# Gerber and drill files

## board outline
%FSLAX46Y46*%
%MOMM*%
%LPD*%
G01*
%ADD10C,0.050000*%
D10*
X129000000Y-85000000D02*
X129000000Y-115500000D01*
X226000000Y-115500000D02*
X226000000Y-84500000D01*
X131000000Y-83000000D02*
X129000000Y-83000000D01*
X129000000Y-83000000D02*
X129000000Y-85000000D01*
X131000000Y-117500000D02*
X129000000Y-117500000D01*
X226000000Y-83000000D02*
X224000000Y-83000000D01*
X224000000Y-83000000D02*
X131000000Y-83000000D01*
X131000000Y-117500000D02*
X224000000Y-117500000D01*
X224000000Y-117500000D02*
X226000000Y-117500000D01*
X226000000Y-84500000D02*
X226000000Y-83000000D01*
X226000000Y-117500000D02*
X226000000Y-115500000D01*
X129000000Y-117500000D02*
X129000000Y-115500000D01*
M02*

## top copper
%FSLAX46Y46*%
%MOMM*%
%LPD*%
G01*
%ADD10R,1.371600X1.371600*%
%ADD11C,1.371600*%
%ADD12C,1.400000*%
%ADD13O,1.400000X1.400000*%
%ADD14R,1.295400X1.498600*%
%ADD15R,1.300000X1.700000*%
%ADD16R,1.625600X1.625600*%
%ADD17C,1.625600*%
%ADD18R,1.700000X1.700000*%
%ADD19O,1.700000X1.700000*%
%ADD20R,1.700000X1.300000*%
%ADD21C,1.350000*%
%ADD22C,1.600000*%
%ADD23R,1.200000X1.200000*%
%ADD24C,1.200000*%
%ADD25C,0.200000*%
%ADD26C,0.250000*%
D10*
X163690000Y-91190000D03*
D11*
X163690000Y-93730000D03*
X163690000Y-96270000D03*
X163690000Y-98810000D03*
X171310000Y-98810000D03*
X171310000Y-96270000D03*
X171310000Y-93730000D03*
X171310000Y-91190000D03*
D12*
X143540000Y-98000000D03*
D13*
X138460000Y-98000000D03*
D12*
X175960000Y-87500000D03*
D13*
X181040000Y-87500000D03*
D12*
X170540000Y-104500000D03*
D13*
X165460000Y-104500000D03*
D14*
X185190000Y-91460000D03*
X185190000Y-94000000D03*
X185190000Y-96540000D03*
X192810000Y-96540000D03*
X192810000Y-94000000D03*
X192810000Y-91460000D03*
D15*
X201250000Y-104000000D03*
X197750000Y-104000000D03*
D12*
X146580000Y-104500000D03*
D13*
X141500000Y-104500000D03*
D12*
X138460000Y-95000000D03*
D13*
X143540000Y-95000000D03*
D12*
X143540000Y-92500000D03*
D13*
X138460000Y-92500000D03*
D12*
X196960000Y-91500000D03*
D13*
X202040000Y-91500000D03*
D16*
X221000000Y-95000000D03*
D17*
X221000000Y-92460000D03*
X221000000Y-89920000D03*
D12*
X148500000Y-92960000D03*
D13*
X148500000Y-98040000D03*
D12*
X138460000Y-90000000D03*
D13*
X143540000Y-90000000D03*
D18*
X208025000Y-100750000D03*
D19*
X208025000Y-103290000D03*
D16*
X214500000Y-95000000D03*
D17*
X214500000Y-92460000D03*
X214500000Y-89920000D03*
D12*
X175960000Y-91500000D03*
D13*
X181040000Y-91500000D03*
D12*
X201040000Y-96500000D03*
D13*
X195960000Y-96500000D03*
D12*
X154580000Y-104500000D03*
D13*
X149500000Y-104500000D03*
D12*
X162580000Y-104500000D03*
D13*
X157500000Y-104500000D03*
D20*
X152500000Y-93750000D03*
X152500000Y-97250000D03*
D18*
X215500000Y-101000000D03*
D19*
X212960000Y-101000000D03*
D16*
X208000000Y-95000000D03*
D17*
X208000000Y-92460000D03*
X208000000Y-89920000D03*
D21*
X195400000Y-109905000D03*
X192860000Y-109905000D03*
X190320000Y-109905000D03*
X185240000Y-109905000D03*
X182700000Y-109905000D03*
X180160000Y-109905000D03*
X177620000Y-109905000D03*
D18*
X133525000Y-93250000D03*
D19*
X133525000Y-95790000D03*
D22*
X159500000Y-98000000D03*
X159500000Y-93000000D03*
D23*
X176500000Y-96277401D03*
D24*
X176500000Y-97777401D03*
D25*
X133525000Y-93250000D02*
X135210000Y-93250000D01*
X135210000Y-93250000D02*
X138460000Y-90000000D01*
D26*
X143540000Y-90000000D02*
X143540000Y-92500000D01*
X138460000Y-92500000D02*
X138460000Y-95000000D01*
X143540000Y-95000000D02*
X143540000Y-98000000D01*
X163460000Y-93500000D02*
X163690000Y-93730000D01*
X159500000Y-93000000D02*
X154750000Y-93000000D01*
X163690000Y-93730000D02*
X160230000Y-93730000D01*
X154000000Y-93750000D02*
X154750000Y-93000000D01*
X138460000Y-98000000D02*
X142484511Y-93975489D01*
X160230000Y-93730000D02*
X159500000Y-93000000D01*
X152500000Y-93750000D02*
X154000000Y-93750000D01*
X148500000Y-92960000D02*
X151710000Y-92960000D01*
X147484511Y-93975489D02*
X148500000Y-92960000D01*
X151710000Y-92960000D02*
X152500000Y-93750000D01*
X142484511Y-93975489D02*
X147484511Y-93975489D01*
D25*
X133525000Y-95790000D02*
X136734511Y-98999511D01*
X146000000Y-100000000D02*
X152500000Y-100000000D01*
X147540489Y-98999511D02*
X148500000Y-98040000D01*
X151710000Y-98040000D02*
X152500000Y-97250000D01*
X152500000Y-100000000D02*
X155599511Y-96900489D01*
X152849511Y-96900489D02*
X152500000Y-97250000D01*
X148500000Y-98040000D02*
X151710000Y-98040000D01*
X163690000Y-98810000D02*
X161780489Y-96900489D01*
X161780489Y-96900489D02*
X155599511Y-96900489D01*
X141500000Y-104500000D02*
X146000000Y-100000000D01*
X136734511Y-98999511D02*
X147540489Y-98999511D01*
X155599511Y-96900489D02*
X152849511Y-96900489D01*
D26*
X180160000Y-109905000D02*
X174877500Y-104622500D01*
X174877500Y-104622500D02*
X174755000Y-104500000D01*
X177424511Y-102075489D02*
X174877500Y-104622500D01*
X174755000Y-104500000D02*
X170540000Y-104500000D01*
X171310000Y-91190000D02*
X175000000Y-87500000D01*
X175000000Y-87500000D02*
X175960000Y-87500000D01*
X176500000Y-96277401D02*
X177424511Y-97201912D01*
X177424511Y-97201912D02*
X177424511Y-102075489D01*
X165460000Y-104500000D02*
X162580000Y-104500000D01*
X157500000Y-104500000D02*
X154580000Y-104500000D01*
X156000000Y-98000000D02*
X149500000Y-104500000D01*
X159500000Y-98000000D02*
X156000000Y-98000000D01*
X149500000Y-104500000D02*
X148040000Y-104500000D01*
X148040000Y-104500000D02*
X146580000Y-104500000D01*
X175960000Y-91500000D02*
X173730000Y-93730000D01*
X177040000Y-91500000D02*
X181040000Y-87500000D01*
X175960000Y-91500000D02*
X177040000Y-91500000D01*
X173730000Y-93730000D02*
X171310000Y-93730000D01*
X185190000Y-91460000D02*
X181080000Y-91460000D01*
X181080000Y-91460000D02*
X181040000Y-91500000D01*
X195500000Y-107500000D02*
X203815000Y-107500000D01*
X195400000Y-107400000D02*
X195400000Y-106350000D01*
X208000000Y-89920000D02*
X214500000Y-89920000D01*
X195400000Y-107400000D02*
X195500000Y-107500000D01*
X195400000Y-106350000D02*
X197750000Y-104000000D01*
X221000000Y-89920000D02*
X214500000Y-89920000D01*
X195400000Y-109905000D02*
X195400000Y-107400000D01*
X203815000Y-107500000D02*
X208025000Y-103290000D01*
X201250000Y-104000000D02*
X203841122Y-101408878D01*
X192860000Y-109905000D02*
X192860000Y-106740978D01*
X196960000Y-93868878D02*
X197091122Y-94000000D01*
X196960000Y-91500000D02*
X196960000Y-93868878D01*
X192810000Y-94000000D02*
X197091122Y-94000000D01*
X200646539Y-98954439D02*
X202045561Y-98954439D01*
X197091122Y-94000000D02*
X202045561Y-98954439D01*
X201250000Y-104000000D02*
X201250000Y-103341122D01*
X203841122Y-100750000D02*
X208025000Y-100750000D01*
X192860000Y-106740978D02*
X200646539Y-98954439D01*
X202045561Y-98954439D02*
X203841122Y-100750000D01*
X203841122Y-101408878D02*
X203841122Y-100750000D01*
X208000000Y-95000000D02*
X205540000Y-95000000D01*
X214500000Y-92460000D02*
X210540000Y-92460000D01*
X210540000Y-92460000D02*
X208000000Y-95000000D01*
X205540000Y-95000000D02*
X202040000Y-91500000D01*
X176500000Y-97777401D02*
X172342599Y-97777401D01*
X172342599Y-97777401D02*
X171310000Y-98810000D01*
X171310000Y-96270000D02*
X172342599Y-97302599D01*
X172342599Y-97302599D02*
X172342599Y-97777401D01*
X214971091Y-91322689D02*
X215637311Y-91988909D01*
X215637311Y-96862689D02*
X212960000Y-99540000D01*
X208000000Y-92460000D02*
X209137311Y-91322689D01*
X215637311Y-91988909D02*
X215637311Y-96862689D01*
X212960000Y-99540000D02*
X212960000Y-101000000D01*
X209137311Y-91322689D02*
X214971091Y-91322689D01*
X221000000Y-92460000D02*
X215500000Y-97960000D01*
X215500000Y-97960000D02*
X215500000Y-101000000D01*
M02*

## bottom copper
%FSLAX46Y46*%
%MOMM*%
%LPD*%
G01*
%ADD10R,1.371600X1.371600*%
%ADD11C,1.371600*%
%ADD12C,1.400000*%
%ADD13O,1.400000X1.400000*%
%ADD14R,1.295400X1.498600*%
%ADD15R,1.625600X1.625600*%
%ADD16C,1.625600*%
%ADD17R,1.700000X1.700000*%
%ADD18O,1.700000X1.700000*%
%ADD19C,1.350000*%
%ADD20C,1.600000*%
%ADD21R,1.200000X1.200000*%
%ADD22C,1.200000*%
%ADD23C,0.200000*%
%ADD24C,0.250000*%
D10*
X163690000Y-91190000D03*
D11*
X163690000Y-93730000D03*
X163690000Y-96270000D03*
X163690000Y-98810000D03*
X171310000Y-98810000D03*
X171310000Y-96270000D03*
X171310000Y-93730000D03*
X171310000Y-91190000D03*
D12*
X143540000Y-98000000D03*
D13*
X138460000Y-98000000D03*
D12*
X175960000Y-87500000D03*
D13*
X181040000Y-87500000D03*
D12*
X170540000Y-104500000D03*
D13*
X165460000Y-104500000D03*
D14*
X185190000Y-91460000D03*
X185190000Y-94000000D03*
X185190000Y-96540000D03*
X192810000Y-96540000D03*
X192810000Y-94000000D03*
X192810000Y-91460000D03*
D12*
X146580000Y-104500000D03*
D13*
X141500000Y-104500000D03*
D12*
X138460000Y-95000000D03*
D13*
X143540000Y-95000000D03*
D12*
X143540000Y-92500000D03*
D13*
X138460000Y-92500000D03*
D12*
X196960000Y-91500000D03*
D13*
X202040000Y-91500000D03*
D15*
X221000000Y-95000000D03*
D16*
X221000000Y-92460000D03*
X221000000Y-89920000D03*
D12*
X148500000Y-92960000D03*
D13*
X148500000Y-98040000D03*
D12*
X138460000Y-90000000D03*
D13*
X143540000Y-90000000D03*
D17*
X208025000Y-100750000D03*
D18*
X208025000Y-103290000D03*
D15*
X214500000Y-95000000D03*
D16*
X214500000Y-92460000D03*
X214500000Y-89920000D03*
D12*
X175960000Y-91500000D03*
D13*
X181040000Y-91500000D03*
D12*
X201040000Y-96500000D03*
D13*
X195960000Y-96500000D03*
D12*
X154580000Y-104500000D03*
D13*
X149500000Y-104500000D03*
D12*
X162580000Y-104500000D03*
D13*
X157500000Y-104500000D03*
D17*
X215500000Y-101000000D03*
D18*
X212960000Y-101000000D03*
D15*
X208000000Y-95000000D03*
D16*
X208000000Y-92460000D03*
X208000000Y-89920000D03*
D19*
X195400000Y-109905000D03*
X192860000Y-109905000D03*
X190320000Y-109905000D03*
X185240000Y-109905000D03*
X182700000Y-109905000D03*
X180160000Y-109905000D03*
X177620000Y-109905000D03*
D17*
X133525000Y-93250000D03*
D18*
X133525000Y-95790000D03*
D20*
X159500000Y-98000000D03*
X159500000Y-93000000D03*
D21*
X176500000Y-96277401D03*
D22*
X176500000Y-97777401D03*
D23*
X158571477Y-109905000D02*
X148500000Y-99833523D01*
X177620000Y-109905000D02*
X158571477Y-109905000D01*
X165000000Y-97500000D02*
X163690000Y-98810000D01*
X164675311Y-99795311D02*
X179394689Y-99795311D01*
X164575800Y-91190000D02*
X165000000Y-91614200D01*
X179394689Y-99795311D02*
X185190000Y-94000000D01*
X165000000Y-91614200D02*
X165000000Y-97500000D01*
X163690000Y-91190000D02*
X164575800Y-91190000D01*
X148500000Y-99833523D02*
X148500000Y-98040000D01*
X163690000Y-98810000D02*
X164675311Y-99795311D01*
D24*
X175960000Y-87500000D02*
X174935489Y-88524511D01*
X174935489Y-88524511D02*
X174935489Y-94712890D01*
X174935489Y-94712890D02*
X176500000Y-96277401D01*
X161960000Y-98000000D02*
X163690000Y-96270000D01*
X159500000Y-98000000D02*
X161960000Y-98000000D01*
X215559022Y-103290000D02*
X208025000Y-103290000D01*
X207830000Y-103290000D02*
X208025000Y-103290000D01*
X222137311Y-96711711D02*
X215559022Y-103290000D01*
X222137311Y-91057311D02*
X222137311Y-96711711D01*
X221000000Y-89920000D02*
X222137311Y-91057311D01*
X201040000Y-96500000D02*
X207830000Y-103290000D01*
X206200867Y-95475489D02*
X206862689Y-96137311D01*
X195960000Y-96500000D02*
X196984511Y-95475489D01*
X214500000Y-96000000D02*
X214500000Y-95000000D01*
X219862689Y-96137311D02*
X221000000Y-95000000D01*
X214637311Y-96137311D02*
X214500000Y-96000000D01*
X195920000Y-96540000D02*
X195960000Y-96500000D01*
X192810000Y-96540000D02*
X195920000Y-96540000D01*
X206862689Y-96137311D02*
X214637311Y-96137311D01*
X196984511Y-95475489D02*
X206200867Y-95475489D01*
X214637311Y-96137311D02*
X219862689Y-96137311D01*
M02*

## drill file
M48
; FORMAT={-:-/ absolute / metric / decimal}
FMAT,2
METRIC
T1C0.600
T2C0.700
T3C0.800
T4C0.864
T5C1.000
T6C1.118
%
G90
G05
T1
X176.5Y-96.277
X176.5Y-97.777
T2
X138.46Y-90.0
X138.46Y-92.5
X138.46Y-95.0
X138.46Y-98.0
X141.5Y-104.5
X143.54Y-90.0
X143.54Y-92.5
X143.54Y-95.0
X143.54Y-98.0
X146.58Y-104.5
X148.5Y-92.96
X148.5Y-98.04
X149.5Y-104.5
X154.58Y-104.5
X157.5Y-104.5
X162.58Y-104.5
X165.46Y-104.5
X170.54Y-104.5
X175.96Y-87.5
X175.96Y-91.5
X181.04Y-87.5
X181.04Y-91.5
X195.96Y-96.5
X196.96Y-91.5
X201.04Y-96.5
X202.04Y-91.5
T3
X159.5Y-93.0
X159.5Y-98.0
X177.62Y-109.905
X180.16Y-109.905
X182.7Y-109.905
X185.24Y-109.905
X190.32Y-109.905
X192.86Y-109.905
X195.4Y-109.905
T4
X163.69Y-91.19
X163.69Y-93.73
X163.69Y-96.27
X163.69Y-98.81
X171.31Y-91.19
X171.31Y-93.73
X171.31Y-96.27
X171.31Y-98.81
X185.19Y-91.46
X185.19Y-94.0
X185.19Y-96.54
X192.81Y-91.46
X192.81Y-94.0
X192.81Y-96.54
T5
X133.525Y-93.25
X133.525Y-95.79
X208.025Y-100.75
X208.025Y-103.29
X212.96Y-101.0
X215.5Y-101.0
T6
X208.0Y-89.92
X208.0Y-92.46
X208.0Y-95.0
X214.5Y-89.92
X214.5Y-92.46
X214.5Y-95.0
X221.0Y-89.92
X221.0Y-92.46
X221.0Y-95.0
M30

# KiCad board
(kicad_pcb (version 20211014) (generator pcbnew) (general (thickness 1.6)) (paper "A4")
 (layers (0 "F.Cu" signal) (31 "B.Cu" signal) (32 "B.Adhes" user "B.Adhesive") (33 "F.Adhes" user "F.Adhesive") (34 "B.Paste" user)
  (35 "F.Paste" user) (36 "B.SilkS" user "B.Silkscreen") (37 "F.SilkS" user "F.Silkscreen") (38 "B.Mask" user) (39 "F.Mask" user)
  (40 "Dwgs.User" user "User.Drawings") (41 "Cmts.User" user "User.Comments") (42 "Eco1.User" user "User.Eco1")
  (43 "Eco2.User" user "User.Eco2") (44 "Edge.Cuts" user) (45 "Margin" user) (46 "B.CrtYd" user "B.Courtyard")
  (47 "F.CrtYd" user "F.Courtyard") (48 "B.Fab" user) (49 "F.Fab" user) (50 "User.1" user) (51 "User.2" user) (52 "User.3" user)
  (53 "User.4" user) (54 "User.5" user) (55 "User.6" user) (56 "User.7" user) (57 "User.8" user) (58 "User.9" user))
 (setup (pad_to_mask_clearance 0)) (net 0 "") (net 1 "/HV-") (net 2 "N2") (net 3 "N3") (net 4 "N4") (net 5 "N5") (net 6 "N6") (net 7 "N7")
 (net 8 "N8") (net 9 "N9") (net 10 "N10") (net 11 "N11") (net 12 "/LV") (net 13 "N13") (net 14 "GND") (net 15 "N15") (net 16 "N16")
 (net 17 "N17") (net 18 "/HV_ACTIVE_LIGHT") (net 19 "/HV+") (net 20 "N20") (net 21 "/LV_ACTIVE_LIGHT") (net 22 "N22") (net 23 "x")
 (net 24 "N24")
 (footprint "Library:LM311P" (layer "F.Cu") (at 163.69 91.19)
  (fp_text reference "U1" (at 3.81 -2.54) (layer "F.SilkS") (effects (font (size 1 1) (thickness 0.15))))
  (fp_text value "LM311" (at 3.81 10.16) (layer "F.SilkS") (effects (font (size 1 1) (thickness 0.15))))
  (pad "1" thru_hole rect (at 0 0) (size 1.3716 1.3716) (drill 0.8636) (layers *.Cu *.Mask) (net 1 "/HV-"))
  (pad "2" thru_hole circle (at 0 2.54) (size 1.3716 1.3716) (drill 0.8636) (layers *.Cu *.Mask) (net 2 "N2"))
  (pad "3" thru_hole circle (at 0 5.08) (size 1.3716 1.3716) (drill 0.8636) (layers *.Cu *.Mask) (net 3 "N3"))
  (pad "4" thru_hole circle (at 0 7.62) (size 1.3716 1.3716) (drill 0.8636) (layers *.Cu *.Mask) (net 1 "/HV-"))
  (pad "5" thru_hole circle (at 7.62 7.62) (size 1.3716 1.3716) (drill 0.8636) (layers *.Cu *.Mask) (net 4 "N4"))
  (pad "6" thru_hole circle (at 7.62 5.08) (size 1.3716 1.3716) (drill 0.8636) (layers *.Cu *.Mask) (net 4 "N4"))
  (pad "7" thru_hole circle (at 7.62 2.54) (size 1.3716 1.3716) (drill 0.8636) (layers *.Cu *.Mask) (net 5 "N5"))
  (pad "8" thru_hole circle (at 7.62 0) (size 1.3716 1.3716) (drill 0.8636) (layers *.Cu *.Mask) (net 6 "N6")))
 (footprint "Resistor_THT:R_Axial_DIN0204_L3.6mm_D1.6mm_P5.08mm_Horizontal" (layer "F.Cu") (at 143.54 98 180)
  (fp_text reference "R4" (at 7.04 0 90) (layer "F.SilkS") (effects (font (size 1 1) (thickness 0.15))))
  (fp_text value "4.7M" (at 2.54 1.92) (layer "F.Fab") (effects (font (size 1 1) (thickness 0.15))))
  (pad "1" thru_hole circle (at 0 0 180) (size 1.4 1.4) (drill 0.7) (layers *.Cu *.Mask) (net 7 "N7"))
  (pad "2" thru_hole oval (at 5.08 0 180) (size 1.4 1.4) (drill 0.7) (layers *.Cu *.Mask) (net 2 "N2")))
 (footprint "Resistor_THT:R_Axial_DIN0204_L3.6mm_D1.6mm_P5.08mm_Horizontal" (layer "F.Cu") (at 175.96 87.5)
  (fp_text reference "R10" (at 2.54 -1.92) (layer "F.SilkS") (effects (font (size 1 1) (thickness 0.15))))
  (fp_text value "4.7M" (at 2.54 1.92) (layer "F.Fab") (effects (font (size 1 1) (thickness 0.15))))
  (pad "1" thru_hole circle (at 0 0) (size 1.4 1.4) (drill 0.7) (layers *.Cu *.Mask) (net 6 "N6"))
  (pad "2" thru_hole oval (at 5.08 0) (size 1.4 1.4) (drill 0.7) (layers *.Cu *.Mask) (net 5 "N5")))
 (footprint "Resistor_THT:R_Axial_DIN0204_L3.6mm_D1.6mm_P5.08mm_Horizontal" (layer "F.Cu") (at 170.54 104.5 180)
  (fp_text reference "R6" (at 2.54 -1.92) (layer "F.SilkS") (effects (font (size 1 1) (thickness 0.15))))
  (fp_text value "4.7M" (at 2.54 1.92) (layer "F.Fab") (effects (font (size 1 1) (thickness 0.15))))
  (pad "1" thru_hole circle (at 0 0 180) (size 1.4 1.4) (drill 0.7) (layers *.Cu *.Mask) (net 6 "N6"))
  (pad "2" thru_hole oval (at 5.08 0 180) (size 1.4 1.4) (drill 0.7) (layers *.Cu *.Mask) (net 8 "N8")))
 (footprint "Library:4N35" (layer "F.Cu") (at 185.19 91.46)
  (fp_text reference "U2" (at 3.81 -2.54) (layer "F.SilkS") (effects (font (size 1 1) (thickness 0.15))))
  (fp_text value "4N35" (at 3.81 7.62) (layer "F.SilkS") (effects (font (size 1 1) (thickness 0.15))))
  (pad "1" thru_hole rect (at 0 0) (size 1.2954 1.4986) (drill 0.8636) (layers *.Cu *.Mask) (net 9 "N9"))
  (pad "2" thru_hole rect (at 0 2.54) (size 1.2954 1.4986) (drill 0.8636) (layers *.Cu *.Mask) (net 1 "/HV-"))
  (pad "3" thru_hole rect (at 0 5.08) (size 1.2954 1.4986) (drill 0.8636) (layers *.Cu *.Mask) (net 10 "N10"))
  (pad "4" thru_hole rect (at 7.62 5.08) (size 1.2954 1.4986) (drill 0.8636) (layers *.Cu *.Mask) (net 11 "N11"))
  (pad "5" thru_hole rect (at 7.62 2.54) (size 1.2954 1.4986) (drill 0.8636) (layers *.Cu *.Mask) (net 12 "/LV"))
  (pad "6" thru_hole rect (at 7.62 0) (size 1.2954 1.4986) (drill 0.8636) (layers *.Cu *.Mask) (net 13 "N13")))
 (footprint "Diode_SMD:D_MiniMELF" (layer "F.Cu") (at 199.5 104 180)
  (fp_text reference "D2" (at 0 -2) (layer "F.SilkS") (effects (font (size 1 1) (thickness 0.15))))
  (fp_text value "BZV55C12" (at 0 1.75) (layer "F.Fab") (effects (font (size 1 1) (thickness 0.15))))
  (pad "1" smd rect (at -1.75 0 180) (size 1.3 1.7) (layers "F.Cu" "F.Paste" "F.Mask") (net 12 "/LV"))
  (pad "2" smd rect (at 1.75 0 180) (size 1.3 1.7) (layers "F.Cu" "F.Paste" "F.Mask") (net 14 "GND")))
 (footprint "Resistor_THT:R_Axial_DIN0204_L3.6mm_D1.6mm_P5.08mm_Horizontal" (layer "F.Cu") (at 146.58 104.5 180)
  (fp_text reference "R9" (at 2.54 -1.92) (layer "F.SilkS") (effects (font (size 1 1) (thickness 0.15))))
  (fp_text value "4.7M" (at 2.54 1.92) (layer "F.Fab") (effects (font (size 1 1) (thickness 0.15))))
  (pad "1" thru_hole circle (at 0 0 180) (size 1.4 1.4) (drill 0.7) (layers *.Cu *.Mask) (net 3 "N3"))
  (pad "2" thru_hole oval (at 5.08 0 180) (size 1.4 1.4) (drill 0.7) (layers *.Cu *.Mask) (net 1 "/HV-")))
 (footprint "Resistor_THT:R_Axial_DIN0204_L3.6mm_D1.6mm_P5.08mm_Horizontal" (layer "F.Cu") (at 138.46 95)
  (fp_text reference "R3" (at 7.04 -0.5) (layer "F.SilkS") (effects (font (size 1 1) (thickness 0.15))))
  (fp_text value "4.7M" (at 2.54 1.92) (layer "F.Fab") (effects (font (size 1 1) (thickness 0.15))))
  (pad "1" thru_hole circle (at 0 0) (size 1.4 1.4) (drill 0.7) (layers *.Cu *.Mask) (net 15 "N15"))
  (pad "2" thru_hole oval (at 5.08 0) (size 1.4 1.4) (drill 0.7) (layers *.Cu *.Mask) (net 7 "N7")))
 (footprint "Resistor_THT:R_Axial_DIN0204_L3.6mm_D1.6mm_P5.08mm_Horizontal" (layer "F.Cu") (at 143.54 92.5 180)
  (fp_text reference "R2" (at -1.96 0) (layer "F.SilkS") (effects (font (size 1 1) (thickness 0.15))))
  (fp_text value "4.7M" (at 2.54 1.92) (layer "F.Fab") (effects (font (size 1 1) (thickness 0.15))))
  (pad "1" thru_hole circle (at 0 0 180) (size 1.4 1.4) (drill 0.7) (layers *.Cu *.Mask) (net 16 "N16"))
  (pad "2" thru_hole oval (at 5.08 0 180) (size 1.4 1.4) (drill 0.7) (layers *.Cu *.Mask) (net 15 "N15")))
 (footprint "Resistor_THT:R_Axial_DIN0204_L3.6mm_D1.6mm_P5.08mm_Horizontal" (layer "F.Cu") (at 196.96 91.5)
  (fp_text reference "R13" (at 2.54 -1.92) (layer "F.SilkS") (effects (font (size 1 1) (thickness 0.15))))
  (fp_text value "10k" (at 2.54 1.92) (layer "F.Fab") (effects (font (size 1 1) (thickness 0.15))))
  (pad "1" thru_hole circle (at 0 0) (size 1.4 1.4) (drill 0.7) (layers *.Cu *.Mask) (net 12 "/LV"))
  (pad "2" thru_hole oval (at 5.08 0) (size 1.4 1.4) (drill 0.7) (layers *.Cu *.Mask) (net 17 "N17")))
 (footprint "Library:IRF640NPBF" (layer "F.Cu") (at 221 95 90)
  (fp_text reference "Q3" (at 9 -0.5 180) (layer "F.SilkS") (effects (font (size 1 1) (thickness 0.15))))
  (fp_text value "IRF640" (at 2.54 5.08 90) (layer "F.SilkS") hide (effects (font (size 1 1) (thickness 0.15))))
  (pad "1" thru_hole rect (at 0 0 90) (size 1.6256 1.6256) (drill 1.1176) (layers *.Cu *.Mask) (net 11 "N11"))
  (pad "2" thru_hole circle (at 2.54 0 90) (size 1.6256 1.6256) (drill 1.1176) (layers *.Cu *.Mask) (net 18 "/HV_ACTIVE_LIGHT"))
  (pad "3" thru_hole circle (at 5.08 0 90) (size 1.6256 1.6256) (drill 1.1176) (layers *.Cu *.Mask) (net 14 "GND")))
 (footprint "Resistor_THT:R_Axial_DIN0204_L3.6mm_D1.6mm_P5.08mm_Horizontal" (layer "F.Cu") (at 148.5 92.96 -90)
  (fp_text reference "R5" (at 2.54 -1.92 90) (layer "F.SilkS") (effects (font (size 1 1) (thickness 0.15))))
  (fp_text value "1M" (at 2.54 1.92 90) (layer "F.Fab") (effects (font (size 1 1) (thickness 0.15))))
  (pad "1" thru_hole circle (at 0 0 270) (size 1.4 1.4) (drill 0.7) (layers *.Cu *.Mask) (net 2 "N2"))
  (pad "2" thru_hole oval (at 5.08 0 270) (size 1.4 1.4) (drill 0.7) (layers *.Cu *.Mask) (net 1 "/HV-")))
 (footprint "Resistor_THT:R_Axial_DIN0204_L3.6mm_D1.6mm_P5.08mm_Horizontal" (layer "F.Cu") (at 138.46 90)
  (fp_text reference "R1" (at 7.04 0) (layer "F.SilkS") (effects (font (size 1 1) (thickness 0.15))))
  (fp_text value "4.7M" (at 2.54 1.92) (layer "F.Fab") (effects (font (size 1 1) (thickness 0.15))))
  (pad "1" thru_hole circle (at 0 0) (size 1.4 1.4) (drill 0.7) (layers *.Cu *.Mask) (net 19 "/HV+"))
  (pad "2" thru_hole oval (at 5.08 0) (size 1.4 1.4) (drill 0.7) (layers *.Cu *.Mask) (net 16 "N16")))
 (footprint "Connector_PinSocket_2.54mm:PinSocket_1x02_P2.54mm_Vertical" (layer "F.Cu") (at 208.025 100.75)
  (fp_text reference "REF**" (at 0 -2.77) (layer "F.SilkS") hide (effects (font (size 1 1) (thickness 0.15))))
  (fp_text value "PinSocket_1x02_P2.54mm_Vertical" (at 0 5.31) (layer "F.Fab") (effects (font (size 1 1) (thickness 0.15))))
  (pad "1" thru_hole rect (at 0 0) (size 1.7 1.7) (drill 1) (layers *.Cu *.Mask) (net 12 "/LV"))
  (pad "2" thru_hole oval (at 0 2.54) (size 1.7 1.7) (drill 1) (layers *.Cu *.Mask) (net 14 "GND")))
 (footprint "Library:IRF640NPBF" (layer "F.Cu") (at 214.5 95 90)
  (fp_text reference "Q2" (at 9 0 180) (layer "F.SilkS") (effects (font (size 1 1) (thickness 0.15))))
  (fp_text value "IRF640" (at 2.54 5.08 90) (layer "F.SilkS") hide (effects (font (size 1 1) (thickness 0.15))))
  (pad "1" thru_hole rect (at 0 0 90) (size 1.6256 1.6256) (drill 1.1176) (layers *.Cu *.Mask) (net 11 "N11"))
  (pad "2" thru_hole circle (at 2.54 0 90) (size 1.6256 1.6256) (drill 1.1176) (layers *.Cu *.Mask) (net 17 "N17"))
  (pad "3" thru_hole circle (at 5.08 0 90) (size 1.6256 1.6256) (drill 1.1176) (layers *.Cu *.Mask) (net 14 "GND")))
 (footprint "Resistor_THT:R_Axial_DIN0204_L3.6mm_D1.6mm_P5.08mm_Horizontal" (layer "F.Cu") (at 175.96 91.5)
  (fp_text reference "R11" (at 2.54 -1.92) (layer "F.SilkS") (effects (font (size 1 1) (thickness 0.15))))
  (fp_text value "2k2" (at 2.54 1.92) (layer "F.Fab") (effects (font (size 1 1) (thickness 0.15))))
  (pad "1" thru_hole circle (at 0 0) (size 1.4 1.4) (drill 0.7) (layers *.Cu *.Mask) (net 5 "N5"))
  (pad "2" thru_hole oval (at 5.08 0) (size 1.4 1.4) (drill 0.7) (layers *.Cu *.Mask) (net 9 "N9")))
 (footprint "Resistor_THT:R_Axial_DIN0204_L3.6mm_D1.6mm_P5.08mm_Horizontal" (layer "F.Cu") (at 201.04 96.5 180)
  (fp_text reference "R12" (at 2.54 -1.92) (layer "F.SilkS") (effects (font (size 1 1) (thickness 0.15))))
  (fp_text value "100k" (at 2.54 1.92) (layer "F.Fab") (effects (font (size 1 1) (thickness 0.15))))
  (pad "1" thru_hole circle (at 0 0 180) (size 1.4 1.4) (drill 0.7) (layers *.Cu *.Mask) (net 14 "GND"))
  (pad "2" thru_hole oval (at 5.08 0 180) (size 1.4 1.4) (drill 0.7) (layers *.Cu *.Mask) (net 11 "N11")))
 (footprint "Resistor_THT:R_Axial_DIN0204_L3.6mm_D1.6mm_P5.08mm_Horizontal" (layer "F.Cu") (at 154.58 104.5 180)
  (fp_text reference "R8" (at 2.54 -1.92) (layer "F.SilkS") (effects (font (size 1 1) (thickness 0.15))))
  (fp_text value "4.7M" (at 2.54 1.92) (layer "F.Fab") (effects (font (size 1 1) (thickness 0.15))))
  (pad "1" thru_hole circle (at 0 0 180) (size 1.4 1.4) (drill 0.7) (layers *.Cu *.Mask) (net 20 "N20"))
  (pad "2" thru_hole oval (at 5.08 0 180) (size 1.4 1.4) (drill 0.7) (layers *.Cu *.Mask) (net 3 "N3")))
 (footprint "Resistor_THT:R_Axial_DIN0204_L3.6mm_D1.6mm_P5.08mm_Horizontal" (layer "F.Cu") (at 162.58 104.5 180)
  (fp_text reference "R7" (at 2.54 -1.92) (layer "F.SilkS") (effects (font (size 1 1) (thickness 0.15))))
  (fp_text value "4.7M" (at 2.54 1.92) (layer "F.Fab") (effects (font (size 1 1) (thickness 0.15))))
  (pad "1" thru_hole circle (at 0 0 180) (size 1.4 1.4) (drill 0.7) (layers *.Cu *.Mask) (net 8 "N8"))
  (pad "2" thru_hole oval (at 5.08 0 180) (size 1.4 1.4) (drill 0.7) (layers *.Cu *.Mask) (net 20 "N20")))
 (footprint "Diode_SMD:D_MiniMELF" (layer "F.Cu") (at 152.5 95.5 -90)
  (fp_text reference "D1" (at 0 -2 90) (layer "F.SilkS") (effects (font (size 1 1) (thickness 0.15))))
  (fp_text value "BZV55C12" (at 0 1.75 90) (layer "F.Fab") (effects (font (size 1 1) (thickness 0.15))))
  (pad "1" smd rect (at -1.75 0 270) (size 1.3 1.7) (layers "F.Cu" "F.Paste" "F.Mask") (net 2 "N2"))
  (pad "2" smd rect (at 1.75 0 270) (size 1.3 1.7) (layers "F.Cu" "F.Paste" "F.Mask") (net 1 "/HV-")))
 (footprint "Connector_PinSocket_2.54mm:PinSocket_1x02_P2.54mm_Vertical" (layer "F.Cu") (at 215.5 101 -90)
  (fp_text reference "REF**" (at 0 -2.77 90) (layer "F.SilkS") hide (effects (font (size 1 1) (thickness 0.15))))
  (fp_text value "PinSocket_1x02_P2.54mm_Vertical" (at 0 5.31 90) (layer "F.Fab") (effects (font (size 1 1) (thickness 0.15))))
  (pad "1" thru_hole rect (at 0 0 270) (size 1.7 1.7) (drill 1) (layers *.Cu *.Mask) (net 18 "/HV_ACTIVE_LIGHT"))
  (pad "2" thru_hole oval (at 0 2.54 270) (size 1.7 1.7) (drill 1) (layers *.Cu *.Mask) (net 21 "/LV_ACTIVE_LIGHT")))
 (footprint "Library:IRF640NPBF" (layer "F.Cu") (at 208 95 90)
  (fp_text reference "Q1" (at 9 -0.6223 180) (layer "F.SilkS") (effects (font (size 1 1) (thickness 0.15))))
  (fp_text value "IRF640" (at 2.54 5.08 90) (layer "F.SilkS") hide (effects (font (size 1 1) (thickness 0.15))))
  (pad "1" thru_hole rect (at 0 0 90) (size 1.6256 1.6256) (drill 1.1176) (layers *.Cu *.Mask) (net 17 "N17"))
  (pad "2" thru_hole circle (at 2.54 0 90) (size 1.6256 1.6256) (drill 1.1176) (layers *.Cu *.Mask) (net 21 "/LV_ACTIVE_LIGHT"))
  (pad "3" thru_hole circle (at 5.08 0 90) (size 1.6256 1.6256) (drill 1.1176) (layers *.Cu *.Mask) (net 14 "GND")))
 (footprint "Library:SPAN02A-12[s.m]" (layer "F.Cu") (at 185.24 97.205 180)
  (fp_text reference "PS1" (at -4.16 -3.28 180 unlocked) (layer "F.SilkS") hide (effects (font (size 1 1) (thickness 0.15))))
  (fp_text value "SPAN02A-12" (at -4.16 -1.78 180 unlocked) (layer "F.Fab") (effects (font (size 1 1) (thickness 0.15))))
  (pad "1" thru_hole circle (at -10.16 -12.7 180) (size 1.35 1.35) (drill 0.8) (layers *.Cu *.Mask) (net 14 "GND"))
  (pad "2" thru_hole circle (at -7.62 -12.7 180) (size 1.35 1.35) (drill 0.8) (layers *.Cu *.Mask) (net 12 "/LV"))
  (pad "3" thru_hole circle (at -5.08 -12.7 180) (size 1.35 1.35) (drill 0.8) (layers *.Cu *.Mask) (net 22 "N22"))
  (pad "4" thru_hole circle (at 0 -12.7 180) (size 1.35 1.35) (drill 0.8) (layers *.Cu *.Mask) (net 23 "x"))
  (pad "5" thru_hole circle (at 2.54 -12.7 180) (size 1.35 1.35) (drill 0.8) (layers *.Cu *.Mask) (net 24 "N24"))
  (pad "6" thru_hole circle (at 5.08 -12.7 180) (size 1.35 1.35) (drill 0.8) (layers *.Cu *.Mask) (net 6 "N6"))
  (pad "7" thru_hole circle (at 7.62 -12.7 180) (size 1.35 1.35) (drill 0.8) (layers *.Cu *.Mask) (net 1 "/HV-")))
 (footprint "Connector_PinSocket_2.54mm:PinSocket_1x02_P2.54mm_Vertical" (layer "F.Cu") (at 133.525 93.25)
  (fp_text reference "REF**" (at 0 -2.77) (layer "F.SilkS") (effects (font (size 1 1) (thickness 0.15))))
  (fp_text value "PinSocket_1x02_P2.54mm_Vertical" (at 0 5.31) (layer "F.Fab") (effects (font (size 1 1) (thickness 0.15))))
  (pad "1" thru_hole rect (at 0 0) (size 1.7 1.7) (drill 1) (layers *.Cu "F.Mask") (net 19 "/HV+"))
  (pad "2" thru_hole oval (at 0 2.54) (size 1.7 1.7) (drill 1) (layers *.Cu *.Mask) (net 1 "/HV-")))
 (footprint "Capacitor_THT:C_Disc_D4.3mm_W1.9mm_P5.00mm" (layer "F.Cu") (at 159.5 98 90)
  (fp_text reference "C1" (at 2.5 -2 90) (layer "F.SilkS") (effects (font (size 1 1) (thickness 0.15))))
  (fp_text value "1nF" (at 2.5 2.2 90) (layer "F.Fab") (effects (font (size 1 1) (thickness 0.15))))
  (pad "1" thru_hole circle (at 0 0 90) (size 1.6 1.6) (drill 0.8) (layers *.Cu *.Mask) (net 3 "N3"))
  (pad "2" thru_hole circle (at 5 0 90) (size 1.6 1.6) (drill 0.8) (layers *.Cu *.Mask) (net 2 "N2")))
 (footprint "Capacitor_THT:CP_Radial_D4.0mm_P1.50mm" (layer "F.Cu") (at 176.5 96.277401 -90)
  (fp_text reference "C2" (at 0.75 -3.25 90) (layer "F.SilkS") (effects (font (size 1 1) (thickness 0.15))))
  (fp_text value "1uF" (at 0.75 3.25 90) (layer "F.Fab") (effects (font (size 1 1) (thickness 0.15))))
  (pad "1" thru_hole rect (at 0 0 270) (size 1.2 1.2) (drill 0.6) (layers *.Cu *.Mask) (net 6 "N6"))
  (pad "2" thru_hole circle (at 1.5 0 270) (size 1.2 1.2) (drill 0.6) (layers *.Cu *.Mask) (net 4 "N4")))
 (gr_line (start 129 85) (end 129 115.5) (layer "Edge.Cuts") (width 0.05))
 (gr_line (start 226 115.5) (end 226 84.5) (layer "Edge.Cuts") (width 0.05))
 (gr_line (start 131 83) (end 129 83) (layer "Edge.Cuts") (width 0.05))
 (gr_line (start 129 83) (end 129 85) (layer "Edge.Cuts") (width 0.05))
 (gr_line (start 131 117.5) (end 129 117.5) (layer "Edge.Cuts") (width 0.05))
 (gr_line (start 226 83) (end 224 83) (layer "Edge.Cuts") (width 0.05))
 (gr_line (start 224 83) (end 131 83) (layer "Edge.Cuts") (width 0.05))
 (gr_line (start 131 117.5) (end 224 117.5) (layer "Edge.Cuts") (width 0.05))
 (gr_line (start 224 117.5) (end 226 117.5) (layer "Edge.Cuts") (width 0.05))
 (gr_line (start 226 84.5) (end 226 83) (layer "Edge.Cuts") (width 0.05))
 (gr_line (start 226 117.5) (end 226 115.5) (layer "Edge.Cuts") (width 0.05))
 (gr_line (start 129 117.5) (end 129 115.5) (layer "Edge.Cuts") (width 0.05))
 (segment (start 133.525 93.25) (end 135.21 93.25) (width 0.2) (layer "F.Cu") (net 19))
 (segment (start 135.21 93.25) (end 138.46 90) (width 0.2) (layer "F.Cu") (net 19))
 (segment (start 143.54 90) (end 143.54 92.5) (width 0.25) (layer "F.Cu") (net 16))
 (segment (start 138.46 92.5) (end 138.46 95) (width 0.25) (layer "F.Cu") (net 15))
 (segment (start 143.54 95) (end 143.54 98) (width 0.25) (layer "F.Cu") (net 7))
 (segment (start 163.46 93.5) (end 163.69 93.73) (width 0.25) (layer "F.Cu") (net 2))
 (segment (start 159.5 93) (end 154.75 93) (width 0.25) (layer "F.Cu") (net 2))
 (segment (start 163.69 93.73) (end 160.23 93.73) (width 0.25) (layer "F.Cu") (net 2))
 (segment (start 154 93.75) (end 154.75 93) (width 0.25) (layer "F.Cu") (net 2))
 (segment (start 138.46 98) (end 142.484511 93.975489) (width 0.25) (layer "F.Cu") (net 2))
 (segment (start 160.23 93.73) (end 159.5 93) (width 0.25) (layer "F.Cu") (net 2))
 (segment (start 152.5 93.75) (end 154 93.75) (width 0.25) (layer "F.Cu") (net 2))
 (segment (start 148.5 92.96) (end 151.71 92.96) (width 0.25) (layer "F.Cu") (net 2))
 (segment (start 147.484511 93.975489) (end 148.5 92.96) (width 0.25) (layer "F.Cu") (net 2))
 (segment (start 151.71 92.96) (end 152.5 93.75) (width 0.25) (layer "F.Cu") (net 2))
 (segment (start 142.484511 93.975489) (end 147.484511 93.975489) (width 0.25) (layer "F.Cu") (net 2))
 (segment (start 133.525 95.79) (end 136.734511 98.999511) (width 0.2) (layer "F.Cu") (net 1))
 (segment (start 146 100) (end 152.5 100) (width 0.2) (layer "F.Cu") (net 1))
 (segment (start 147.540489 98.999511) (end 148.5 98.04) (width 0.2) (layer "F.Cu") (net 1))
 (segment (start 151.71 98.04) (end 152.5 97.25) (width 0.2) (layer "F.Cu") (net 1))
 (segment (start 152.5 100) (end 155.599511 96.900489) (width 0.2) (layer "F.Cu") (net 1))
 (segment (start 152.849511 96.900489) (end 152.5 97.25) (width 0.2) (layer "F.Cu") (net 1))
 (segment (start 148.5 98.04) (end 151.71 98.04) (width 0.2) (layer "F.Cu") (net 1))
 (segment (start 163.69 98.81) (end 161.780489 96.900489) (width 0.2) (layer "F.Cu") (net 1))
 (segment (start 161.780489 96.900489) (end 155.599511 96.900489) (width 0.2) (layer "F.Cu") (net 1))
 (segment (start 141.5 104.5) (end 146 100) (width 0.2) (layer "F.Cu") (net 1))
 (segment (start 136.734511 98.999511) (end 147.540489 98.999511) (width 0.2) (layer "F.Cu") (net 1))
 (segment (start 155.599511 96.900489) (end 152.849511 96.900489) (width 0.2) (layer "F.Cu") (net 1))
 (segment (start 158.571477 109.905) (end 148.5 99.833523) (width 0.2) (layer "B.Cu") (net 1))
 (segment (start 177.62 109.905) (end 158.571477 109.905) (width 0.2) (layer "B.Cu") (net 1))
 (segment (start 165 97.5) (end 163.69 98.81) (width 0.2) (layer "B.Cu") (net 1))
 (segment (start 164.675311 99.795311) (end 179.394689 99.795311) (width 0.2) (layer "B.Cu") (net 1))
 (segment (start 164.5758 91.19) (end 165 91.6142) (width 0.2) (layer "B.Cu") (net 1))
 (segment (start 179.394689 99.795311) (end 185.19 94) (width 0.2) (layer "B.Cu") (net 1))
 (segment (start 165 91.6142) (end 165 97.5) (width 0.2) (layer "B.Cu") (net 1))
 (segment (start 163.69 91.19) (end 164.5758 91.19) (width 0.2) (layer "B.Cu") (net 1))
 (segment (start 148.5 99.833523) (end 148.5 98.04) (width 0.2) (layer "B.Cu") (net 1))
 (segment (start 163.69 98.81) (end 164.675311 99.795311) (width 0.2) (layer "B.Cu") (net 1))
 (segment (start 180.16 109.905) (end 174.8775 104.6225) (width 0.25) (layer "F.Cu") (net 6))
 (segment (start 174.8775 104.6225) (end 174.755 104.5) (width 0.25) (layer "F.Cu") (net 6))
 (segment (start 177.424511 102.075489) (end 174.8775 104.6225) (width 0.25) (layer "F.Cu") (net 6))
 (segment (start 174.755 104.5) (end 170.54 104.5) (width 0.25) (layer "F.Cu") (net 6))
 (segment (start 171.31 91.19) (end 175 87.5) (width 0.25) (layer "F.Cu") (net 6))
 (segment (start 175 87.5) (end 175.96 87.5) (width 0.25) (layer "F.Cu") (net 6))
 (segment (start 176.5 96.277401) (end 177.424511 97.201912) (width 0.25) (layer "F.Cu") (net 6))
 (segment (start 177.424511 97.201912) (end 177.424511 102.075489) (width 0.25) (layer "F.Cu") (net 6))
 (segment (start 175.96 87.5) (end 174.935489 88.524511) (width 0.25) (layer "B.Cu") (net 6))
 (segment (start 174.935489 88.524511) (end 174.935489 94.71289) (width 0.25) (layer "B.Cu") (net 6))
 (segment (start 174.935489 94.71289) (end 176.5 96.277401) (width 0.25) (layer "B.Cu") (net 6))
 (segment (start 165.46 104.5) (end 162.58 104.5) (width 0.25) (layer "F.Cu") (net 8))
 (segment (start 157.5 104.5) (end 154.58 104.5) (width 0.25) (layer "F.Cu") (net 20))
 (segment (start 156 98) (end 149.5 104.5) (width 0.25) (layer "F.Cu") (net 3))
 (segment (start 159.5 98) (end 156 98) (width 0.25) (layer "F.Cu") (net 3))
 (segment (start 149.5 104.5) (end 148.04 104.5) (width 0.25) (layer "F.Cu") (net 3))
 (segment (start 148.04 104.5) (end 146.58 104.5) (width 0.25) (layer "F.Cu") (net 3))
 (segment (start 161.96 98) (end 163.69 96.27) (width 0.25) (layer "B.Cu") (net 3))
 (segment (start 159.5 98) (end 161.96 98) (width 0.25) (layer "B.Cu") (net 3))
 (segment (start 175.96 91.5) (end 173.73 93.73) (width 0.25) (layer "F.Cu") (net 5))
 (segment (start 177.04 91.5) (end 181.04 87.5) (width 0.25) (layer "F.Cu") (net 5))
 (segment (start 175.96 91.5) (end 177.04 91.5) (width 0.25) (layer "F.Cu") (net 5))
 (segment (start 173.73 93.73) (end 171.31 93.73) (width 0.25) (layer "F.Cu") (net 5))
 (segment (start 185.19 91.46) (end 181.08 91.46) (width 0.25) (layer "F.Cu") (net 9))
 (segment (start 181.08 91.46) (end 181.04 91.5) (width 0.25) (layer "F.Cu") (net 9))
 (segment (start 195.5 107.5) (end 203.815 107.5) (width 0.25) (layer "F.Cu") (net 14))
 (segment (start 195.4 107.4) (end 195.4 106.35) (width 0.25) (layer "F.Cu") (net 14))
 (segment (start 208 89.92) (end 214.5 89.92) (width 0.25) (layer "F.Cu") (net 14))
 (segment (start 195.4 107.4) (end 195.5 107.5) (width 0.25) (layer "F.Cu") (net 14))
 (segment (start 195.4 106.35) (end 197.75 104) (width 0.25) (layer "F.Cu") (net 14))
 (segment (start 221 89.92) (end 214.5 89.92) (width 0.25) (layer "F.Cu") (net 14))
 (segment (start 195.4 109.905) (end 195.4 107.4) (width 0.25) (layer "F.Cu") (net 14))
 (segment (start 203.815 107.5) (end 208.025 103.29) (width 0.25) (layer "F.Cu") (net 14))
 (segment (start 215.559022 103.29) (end 208.025 103.29) (width 0.25) (layer "B.Cu") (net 14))
 (segment (start 207.83 103.29) (end 208.025 103.29) (width 0.25) (layer "B.Cu") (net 14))
 (segment (start 222.137311 96.711711) (end 215.559022 103.29) (width 0.25) (layer "B.Cu") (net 14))
 (segment (start 222.137311 91.057311) (end 222.137311 96.711711) (width 0.25) (layer "B.Cu") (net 14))
 (segment (start 221 89.92) (end 222.137311 91.057311) (width 0.25) (layer "B.Cu") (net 14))
 (segment (start 201.04 96.5) (end 207.83 103.29) (width 0.25) (layer "B.Cu") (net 14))
 (segment (start 206.200867 95.475489) (end 206.862689 96.137311) (width 0.25) (layer "B.Cu") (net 11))
 (segment (start 195.96 96.5) (end 196.984511 95.475489) (width 0.25) (layer "B.Cu") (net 11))
 (segment (start 214.5 96) (end 214.5 95) (width 0.25) (layer "B.Cu") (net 11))
 (segment (start 219.862689 96.137311) (end 221 95) (width 0.25) (layer "B.Cu") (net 11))
 (segment (start 214.637311 96.137311) (end 214.5 96) (width 0.25) (layer "B.Cu") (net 11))
 (segment (start 195.92 96.54) (end 195.96 96.5) (width 0.25) (layer "B.Cu") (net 11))
 (segment (start 192.81 96.54) (end 195.92 96.54) (width 0.25) (layer "B.Cu") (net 11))
 (segment (start 206.862689 96.137311) (end 214.637311 96.137311) (width 0.25) (layer "B.Cu") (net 11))
 (segment (start 196.984511 95.475489) (end 206.200867 95.475489) (width 0.25) (layer "B.Cu") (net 11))
 (segment (start 214.637311 96.137311) (end 219.862689 96.137311) (width 0.25) (layer "B.Cu") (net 11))
 (segment (start 201.25 104) (end 203.841122 101.408878) (width 0.25) (layer "F.Cu") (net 12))
 (segment (start 192.86 109.905) (end 192.86 106.740978) (width 0.25) (layer "F.Cu") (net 12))
 (segment (start 196.96 93.868878) (end 197.091122 94) (width 0.25) (layer "F.Cu") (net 12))
 (segment (start 196.96 91.5) (end 196.96 93.868878) (width 0.25) (layer "F.Cu") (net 12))
 (segment (start 192.81 94) (end 197.091122 94) (width 0.25) (layer "F.Cu") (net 12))
 (segment (start 200.646539 98.954439) (end 202.045561 98.954439) (width 0.25) (layer "F.Cu") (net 12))
 (segment (start 197.091122 94) (end 202.045561 98.954439) (width 0.25) (layer "F.Cu") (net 12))
 (segment (start 201.25 104) (end 201.25 103.341122) (width 0.25) (layer "F.Cu") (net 12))
 (segment (start 203.841122 100.75) (end 208.025 100.75) (width 0.25) (layer "F.Cu") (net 12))
 (segment (start 192.86 106.740978) (end 200.646539 98.954439) (width 0.25) (layer "F.Cu") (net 12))
 (segment (start 202.045561 98.954439) (end 203.841122 100.75) (width 0.25) (layer "F.Cu") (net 12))
 (segment (start 203.841122 101.408878) (end 203.841122 100.75) (width 0.25) (layer "F.Cu") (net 12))
 (segment (start 208 95) (end 205.54 95) (width 0.25) (layer "F.Cu") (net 17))
 (segment (start 214.5 92.46) (end 210.54 92.46) (width 0.25) (layer "F.Cu") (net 17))
 (segment (start 210.54 92.46) (end 208 95) (width 0.25) (layer "F.Cu") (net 17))
 (segment (start 205.54 95) (end 202.04 91.5) (width 0.25) (layer "F.Cu") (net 17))
 (segment (start 176.5 97.777401) (end 172.342599 97.777401) (width 0.25) (layer "F.Cu") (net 4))
 (segment (start 172.342599 97.777401) (end 171.31 98.81) (width 0.25) (layer "F.Cu") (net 4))
 (segment (start 171.31 96.27) (end 172.342599 97.302599) (width 0.25) (layer "F.Cu") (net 4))
 (segment (start 172.342599 97.302599) (end 172.342599 97.777401) (width 0.25) (layer "F.Cu") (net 4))
 (segment (start 214.971091 91.322689) (end 215.637311 91.988909) (width 0.25) (layer "F.Cu") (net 21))
 (segment (start 215.637311 96.862689) (end 212.96 99.54) (width 0.25) (layer "F.Cu") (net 21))
 (segment (start 208 92.46) (end 209.137311 91.322689) (width 0.25) (layer "F.Cu") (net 21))
 (segment (start 215.637311 91.988909) (end 215.637311 96.862689) (width 0.25) (layer "F.Cu") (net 21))
 (segment (start 212.96 99.54) (end 212.96 101) (width 0.25) (layer "F.Cu") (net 21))
 (segment (start 209.137311 91.322689) (end 214.971091 91.322689) (width 0.25) (layer "F.Cu") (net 21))
 (segment (start 221 92.46) (end 215.5 97.96) (width 0.25) (layer "F.Cu") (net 18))
 (segment (start 215.5 97.96) (end 215.5 101) (width 0.25) (layer "F.Cu") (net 18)))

